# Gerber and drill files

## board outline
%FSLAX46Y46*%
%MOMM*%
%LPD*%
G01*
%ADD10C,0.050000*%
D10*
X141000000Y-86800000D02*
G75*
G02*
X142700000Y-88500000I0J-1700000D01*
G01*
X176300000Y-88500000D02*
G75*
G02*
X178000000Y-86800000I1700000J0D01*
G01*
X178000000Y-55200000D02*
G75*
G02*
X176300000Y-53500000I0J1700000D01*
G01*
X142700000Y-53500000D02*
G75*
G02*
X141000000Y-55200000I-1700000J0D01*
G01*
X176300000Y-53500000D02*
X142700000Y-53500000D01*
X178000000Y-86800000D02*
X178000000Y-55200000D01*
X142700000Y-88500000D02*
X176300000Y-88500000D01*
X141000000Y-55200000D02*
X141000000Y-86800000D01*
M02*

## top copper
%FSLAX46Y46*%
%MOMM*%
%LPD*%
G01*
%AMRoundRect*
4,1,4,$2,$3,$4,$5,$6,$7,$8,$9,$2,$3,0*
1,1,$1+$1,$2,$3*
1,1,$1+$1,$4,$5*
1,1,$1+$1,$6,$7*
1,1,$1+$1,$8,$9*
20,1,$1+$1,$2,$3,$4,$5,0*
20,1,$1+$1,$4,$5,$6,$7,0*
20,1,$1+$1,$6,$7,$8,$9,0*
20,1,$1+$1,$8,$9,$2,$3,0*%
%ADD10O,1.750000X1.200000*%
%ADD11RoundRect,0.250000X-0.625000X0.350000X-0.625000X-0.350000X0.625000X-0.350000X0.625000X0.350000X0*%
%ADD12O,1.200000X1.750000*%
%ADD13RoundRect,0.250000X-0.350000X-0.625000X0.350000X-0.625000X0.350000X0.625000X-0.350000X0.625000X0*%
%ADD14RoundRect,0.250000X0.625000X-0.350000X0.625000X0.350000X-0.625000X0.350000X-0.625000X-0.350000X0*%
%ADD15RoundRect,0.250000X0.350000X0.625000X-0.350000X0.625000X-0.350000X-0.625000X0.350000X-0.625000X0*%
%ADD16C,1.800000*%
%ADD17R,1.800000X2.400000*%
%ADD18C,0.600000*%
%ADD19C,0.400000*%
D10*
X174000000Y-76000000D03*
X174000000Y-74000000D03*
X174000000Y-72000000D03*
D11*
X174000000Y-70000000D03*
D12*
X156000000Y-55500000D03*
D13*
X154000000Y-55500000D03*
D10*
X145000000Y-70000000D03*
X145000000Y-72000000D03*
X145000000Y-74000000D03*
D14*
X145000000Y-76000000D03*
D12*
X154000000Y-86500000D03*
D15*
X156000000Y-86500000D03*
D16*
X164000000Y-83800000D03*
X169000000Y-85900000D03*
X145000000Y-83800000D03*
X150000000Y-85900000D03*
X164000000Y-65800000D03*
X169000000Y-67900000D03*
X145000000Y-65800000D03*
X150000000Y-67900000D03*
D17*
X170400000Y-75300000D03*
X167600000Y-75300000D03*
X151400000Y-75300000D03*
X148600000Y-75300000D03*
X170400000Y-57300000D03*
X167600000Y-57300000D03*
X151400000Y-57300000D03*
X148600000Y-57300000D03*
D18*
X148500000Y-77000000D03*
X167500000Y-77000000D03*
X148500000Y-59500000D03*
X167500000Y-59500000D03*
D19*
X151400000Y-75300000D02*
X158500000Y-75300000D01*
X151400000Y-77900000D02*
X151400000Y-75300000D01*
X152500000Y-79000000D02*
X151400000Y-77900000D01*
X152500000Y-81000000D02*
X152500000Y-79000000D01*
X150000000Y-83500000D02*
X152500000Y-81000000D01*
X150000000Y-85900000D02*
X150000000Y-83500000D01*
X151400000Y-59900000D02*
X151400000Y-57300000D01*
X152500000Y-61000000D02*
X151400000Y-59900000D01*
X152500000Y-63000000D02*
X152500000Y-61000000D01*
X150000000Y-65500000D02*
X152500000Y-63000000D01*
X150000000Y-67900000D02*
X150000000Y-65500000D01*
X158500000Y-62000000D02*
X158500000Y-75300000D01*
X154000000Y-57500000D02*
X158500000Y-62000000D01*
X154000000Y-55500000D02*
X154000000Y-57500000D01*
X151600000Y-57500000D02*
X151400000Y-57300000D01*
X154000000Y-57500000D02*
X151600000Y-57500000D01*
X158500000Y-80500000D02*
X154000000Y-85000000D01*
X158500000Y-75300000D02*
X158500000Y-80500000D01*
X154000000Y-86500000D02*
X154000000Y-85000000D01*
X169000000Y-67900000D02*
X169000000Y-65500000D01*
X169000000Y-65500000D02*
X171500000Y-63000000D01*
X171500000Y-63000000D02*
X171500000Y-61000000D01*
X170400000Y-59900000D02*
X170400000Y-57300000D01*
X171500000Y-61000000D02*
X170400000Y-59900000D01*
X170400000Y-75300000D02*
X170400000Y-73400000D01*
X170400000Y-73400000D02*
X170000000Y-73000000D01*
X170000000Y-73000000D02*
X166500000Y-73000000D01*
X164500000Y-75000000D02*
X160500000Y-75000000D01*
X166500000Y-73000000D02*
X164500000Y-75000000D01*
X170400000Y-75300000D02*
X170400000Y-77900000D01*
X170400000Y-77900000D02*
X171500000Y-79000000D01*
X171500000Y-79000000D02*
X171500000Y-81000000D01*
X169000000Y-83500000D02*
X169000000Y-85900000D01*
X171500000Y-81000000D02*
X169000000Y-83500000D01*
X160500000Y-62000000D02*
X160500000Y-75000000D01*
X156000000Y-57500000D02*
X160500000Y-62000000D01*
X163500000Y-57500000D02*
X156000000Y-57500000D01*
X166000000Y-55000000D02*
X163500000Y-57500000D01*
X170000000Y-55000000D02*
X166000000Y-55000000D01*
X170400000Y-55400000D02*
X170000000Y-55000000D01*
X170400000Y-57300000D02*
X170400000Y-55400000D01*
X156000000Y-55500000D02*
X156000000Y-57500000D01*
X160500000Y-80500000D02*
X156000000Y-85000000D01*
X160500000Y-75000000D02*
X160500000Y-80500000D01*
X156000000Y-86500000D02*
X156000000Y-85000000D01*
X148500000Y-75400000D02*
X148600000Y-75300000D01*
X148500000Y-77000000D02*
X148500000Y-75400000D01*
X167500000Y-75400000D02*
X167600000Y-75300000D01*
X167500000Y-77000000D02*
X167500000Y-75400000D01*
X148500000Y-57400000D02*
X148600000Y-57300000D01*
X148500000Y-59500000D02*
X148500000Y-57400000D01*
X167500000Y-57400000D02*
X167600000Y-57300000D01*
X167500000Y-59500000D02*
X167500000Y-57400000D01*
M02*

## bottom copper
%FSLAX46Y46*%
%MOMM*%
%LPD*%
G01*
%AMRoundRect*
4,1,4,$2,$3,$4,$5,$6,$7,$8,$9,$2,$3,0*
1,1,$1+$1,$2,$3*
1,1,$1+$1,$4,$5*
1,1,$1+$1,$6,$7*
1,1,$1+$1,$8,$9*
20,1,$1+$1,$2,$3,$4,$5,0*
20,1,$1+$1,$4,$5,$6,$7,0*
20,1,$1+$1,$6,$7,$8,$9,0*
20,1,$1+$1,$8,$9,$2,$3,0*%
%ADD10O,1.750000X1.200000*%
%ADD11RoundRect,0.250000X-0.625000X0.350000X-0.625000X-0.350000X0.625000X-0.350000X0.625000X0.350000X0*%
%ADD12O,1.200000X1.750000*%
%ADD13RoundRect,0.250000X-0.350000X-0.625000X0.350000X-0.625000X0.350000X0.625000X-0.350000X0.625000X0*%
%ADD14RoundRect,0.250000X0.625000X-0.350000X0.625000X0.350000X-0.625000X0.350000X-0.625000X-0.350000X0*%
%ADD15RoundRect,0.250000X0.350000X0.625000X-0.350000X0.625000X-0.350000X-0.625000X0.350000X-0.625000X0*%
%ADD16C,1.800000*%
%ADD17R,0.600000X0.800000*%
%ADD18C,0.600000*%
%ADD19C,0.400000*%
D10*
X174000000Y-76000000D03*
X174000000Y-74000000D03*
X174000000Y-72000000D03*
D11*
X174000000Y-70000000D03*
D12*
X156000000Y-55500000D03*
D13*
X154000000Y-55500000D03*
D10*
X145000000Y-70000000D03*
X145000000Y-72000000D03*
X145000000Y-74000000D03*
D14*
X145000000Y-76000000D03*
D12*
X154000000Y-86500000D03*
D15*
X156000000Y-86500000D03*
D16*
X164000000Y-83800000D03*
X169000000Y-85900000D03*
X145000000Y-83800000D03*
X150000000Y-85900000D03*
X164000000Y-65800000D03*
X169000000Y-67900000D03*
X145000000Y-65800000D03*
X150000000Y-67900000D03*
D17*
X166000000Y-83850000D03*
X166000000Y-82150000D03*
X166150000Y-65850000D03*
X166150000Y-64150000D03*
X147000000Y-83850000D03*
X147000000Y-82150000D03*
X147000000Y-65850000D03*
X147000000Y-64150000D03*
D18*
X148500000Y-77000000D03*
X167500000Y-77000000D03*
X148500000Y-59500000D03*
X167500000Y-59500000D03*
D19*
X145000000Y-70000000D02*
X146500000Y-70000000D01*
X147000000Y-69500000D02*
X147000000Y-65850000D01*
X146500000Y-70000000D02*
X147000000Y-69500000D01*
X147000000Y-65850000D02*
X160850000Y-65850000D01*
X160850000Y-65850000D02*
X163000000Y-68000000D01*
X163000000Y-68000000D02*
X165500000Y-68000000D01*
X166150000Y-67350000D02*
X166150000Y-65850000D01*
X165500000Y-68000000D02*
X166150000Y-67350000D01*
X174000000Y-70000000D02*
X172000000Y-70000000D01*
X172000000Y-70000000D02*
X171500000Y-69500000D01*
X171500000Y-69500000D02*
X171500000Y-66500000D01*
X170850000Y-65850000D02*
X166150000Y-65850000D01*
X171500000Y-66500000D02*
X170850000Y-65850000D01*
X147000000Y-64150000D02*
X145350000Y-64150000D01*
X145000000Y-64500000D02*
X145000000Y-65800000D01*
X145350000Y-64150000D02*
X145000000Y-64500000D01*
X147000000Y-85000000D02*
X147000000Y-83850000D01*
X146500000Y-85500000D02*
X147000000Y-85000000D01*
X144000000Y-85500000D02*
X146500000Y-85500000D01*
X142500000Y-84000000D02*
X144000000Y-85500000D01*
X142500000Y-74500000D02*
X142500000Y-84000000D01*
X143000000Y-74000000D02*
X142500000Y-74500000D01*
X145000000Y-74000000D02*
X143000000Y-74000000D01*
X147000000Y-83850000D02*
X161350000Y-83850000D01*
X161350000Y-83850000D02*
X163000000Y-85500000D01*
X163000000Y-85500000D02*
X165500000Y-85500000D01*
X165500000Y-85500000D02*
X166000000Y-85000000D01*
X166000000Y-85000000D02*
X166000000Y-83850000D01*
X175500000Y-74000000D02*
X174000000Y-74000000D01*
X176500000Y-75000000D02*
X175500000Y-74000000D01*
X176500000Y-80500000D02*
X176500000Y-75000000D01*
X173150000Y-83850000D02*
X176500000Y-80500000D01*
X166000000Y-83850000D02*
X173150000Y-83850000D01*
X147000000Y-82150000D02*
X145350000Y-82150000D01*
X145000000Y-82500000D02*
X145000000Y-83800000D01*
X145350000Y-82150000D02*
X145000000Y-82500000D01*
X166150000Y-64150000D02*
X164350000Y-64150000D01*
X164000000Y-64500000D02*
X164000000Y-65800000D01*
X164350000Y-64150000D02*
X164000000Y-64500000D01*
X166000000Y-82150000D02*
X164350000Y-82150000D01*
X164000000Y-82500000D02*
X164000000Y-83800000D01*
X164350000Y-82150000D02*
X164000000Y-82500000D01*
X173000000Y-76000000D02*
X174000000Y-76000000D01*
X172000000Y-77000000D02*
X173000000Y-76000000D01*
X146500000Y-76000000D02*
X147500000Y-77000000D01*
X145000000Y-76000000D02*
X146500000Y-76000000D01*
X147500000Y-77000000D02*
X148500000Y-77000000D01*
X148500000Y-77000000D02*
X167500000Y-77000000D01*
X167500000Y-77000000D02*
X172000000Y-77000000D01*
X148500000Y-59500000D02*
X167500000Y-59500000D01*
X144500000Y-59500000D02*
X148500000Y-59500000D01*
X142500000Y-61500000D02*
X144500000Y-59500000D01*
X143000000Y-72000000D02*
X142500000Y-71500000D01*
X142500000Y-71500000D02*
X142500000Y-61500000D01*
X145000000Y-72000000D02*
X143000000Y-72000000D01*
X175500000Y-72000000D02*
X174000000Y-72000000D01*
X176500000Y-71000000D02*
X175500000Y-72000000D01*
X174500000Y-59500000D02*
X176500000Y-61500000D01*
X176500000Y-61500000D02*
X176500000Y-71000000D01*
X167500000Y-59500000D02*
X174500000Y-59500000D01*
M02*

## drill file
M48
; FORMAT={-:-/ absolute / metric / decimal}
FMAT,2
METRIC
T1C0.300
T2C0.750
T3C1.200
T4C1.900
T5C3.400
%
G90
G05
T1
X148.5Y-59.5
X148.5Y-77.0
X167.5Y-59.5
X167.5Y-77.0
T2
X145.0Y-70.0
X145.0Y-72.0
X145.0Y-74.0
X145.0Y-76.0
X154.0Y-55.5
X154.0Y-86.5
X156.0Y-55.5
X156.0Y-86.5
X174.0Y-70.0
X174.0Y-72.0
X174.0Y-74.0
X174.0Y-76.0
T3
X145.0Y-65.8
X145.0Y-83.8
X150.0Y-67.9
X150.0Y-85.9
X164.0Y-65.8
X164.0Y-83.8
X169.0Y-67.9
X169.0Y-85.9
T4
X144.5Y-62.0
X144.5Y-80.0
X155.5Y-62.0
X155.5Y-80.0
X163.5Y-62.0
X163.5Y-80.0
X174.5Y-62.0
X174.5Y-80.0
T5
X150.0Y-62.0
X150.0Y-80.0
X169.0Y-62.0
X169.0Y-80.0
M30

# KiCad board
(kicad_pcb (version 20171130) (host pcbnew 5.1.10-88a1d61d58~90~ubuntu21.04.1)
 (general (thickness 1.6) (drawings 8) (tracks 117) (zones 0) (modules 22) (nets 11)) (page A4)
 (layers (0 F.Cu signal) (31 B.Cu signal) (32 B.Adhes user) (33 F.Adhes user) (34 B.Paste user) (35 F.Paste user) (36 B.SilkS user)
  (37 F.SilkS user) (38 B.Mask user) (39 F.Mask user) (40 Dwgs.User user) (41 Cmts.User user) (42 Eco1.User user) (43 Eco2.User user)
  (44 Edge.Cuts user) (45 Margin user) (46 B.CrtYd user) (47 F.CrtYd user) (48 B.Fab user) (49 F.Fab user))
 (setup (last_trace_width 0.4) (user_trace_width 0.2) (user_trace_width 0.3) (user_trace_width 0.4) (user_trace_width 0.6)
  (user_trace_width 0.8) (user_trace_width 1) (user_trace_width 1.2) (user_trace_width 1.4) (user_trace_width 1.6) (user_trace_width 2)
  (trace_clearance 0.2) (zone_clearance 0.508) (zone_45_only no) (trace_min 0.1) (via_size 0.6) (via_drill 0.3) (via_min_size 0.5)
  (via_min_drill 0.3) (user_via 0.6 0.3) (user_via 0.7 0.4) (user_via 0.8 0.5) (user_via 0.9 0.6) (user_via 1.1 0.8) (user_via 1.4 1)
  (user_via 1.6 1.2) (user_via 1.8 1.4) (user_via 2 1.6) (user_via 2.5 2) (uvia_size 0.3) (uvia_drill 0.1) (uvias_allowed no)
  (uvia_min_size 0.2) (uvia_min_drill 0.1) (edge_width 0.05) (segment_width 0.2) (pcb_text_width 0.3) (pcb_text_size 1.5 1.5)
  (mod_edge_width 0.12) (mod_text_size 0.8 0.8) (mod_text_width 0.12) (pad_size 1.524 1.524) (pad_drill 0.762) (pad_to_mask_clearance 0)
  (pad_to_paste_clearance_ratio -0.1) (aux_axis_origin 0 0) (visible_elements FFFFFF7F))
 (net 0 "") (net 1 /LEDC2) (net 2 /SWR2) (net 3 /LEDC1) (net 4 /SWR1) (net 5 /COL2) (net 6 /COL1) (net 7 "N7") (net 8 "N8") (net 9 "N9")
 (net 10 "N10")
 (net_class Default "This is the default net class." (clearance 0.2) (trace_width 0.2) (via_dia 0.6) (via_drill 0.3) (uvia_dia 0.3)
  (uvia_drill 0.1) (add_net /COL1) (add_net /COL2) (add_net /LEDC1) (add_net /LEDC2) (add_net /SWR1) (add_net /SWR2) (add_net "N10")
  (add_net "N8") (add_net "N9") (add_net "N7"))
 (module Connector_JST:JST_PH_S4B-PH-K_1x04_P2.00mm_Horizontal (layer B.Cu) (at 174 70 270)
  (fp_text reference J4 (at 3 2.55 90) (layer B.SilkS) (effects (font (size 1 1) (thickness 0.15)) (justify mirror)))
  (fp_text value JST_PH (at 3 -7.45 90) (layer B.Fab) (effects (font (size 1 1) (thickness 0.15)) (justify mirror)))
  (pad 4 thru_hole oval (at 6 0 270) (size 1.2 1.75) (drill 0.75) (layers *.Cu *.Mask) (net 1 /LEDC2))
  (pad 3 thru_hole oval (at 4 0 270) (size 1.2 1.75) (drill 0.75) (layers *.Cu *.Mask) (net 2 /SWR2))
  (pad 2 thru_hole oval (at 2 0 270) (size 1.2 1.75) (drill 0.75) (layers *.Cu *.Mask) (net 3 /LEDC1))
  (pad 1 thru_hole roundrect (at 0 0 270) (size 1.2 1.75) (drill 0.75) (layers *.Cu *.Mask) (roundrect_rratio 0.208333) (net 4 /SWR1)))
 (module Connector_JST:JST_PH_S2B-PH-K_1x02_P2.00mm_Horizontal (layer B.Cu) (at 154 55.5)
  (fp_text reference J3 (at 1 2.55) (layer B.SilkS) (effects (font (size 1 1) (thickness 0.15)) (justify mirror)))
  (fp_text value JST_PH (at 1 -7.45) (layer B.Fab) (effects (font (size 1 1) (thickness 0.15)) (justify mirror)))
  (pad 2 thru_hole oval (at 2 0) (size 1.2 1.75) (drill 0.75) (layers *.Cu *.Mask) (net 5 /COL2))
  (pad 1 thru_hole roundrect (at 0 0) (size 1.2 1.75) (drill 0.75) (layers *.Cu *.Mask) (roundrect_rratio 0.208333) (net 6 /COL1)))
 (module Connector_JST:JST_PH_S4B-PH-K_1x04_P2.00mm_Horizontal (layer B.Cu) (at 145 76 90)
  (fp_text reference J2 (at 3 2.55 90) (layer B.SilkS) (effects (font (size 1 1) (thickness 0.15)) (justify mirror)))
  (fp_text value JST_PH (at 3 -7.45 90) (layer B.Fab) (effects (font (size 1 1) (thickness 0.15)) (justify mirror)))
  (pad 4 thru_hole oval (at 6 0 90) (size 1.2 1.75) (drill 0.75) (layers *.Cu *.Mask) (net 4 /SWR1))
  (pad 3 thru_hole oval (at 4 0 90) (size 1.2 1.75) (drill 0.75) (layers *.Cu *.Mask) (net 3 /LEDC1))
  (pad 2 thru_hole oval (at 2 0 90) (size 1.2 1.75) (drill 0.75) (layers *.Cu *.Mask) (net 2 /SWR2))
  (pad 1 thru_hole roundrect (at 0 0 90) (size 1.2 1.75) (drill 0.75) (layers *.Cu *.Mask) (roundrect_rratio 0.208333) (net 1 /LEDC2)))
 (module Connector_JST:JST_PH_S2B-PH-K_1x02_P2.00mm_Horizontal (layer B.Cu) (at 156 86.5 180)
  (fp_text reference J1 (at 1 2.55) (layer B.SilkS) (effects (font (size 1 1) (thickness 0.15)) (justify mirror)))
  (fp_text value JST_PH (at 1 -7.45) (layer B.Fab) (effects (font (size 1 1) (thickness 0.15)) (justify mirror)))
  (pad 2 thru_hole oval (at 2 0 180) (size 1.2 1.75) (drill 0.75) (layers *.Cu *.Mask) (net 6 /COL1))
  (pad 1 thru_hole roundrect (at 0 0 180) (size 1.2 1.75) (drill 0.75) (layers *.Cu *.Mask) (roundrect_rratio 0.208333) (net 5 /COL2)))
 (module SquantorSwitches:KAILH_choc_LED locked (layer F.Cu) (at 169 80 180)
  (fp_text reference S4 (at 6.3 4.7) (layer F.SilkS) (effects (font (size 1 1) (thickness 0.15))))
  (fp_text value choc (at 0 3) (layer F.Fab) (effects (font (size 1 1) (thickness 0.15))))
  (pad 2 thru_hole circle (at 5 -3.8 180) (size 1.8 1.8) (drill 1.2) (layers *.Cu *.Mask) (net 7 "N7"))
  (pad 1 thru_hole circle (at 0 -5.9 180) (size 1.8 1.8) (drill 1.2) (layers *.Cu *.Mask) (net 5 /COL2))
  (pad "" np_thru_hole circle (at 5.5 0 180) (size 1.9 1.9) (drill 1.9) (layers *.Cu *.Mask))
  (pad "" np_thru_hole circle (at -5.5 0 180) (size 1.9 1.9) (drill 1.9) (layers *.Cu *.Mask))
  (pad "" np_thru_hole circle (at 0 0 180) (size 3.4 3.4) (drill 3.4) (layers *.Cu *.Mask)))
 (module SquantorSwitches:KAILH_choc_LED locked (layer F.Cu) (at 150 80 180)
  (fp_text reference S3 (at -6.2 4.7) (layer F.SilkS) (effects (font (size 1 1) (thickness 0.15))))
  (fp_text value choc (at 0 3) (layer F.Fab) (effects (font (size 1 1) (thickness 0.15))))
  (pad 2 thru_hole circle (at 5 -3.8 180) (size 1.8 1.8) (drill 1.2) (layers *.Cu *.Mask) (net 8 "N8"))
  (pad 1 thru_hole circle (at 0 -5.9 180) (size 1.8 1.8) (drill 1.2) (layers *.Cu *.Mask) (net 6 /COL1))
  (pad "" np_thru_hole circle (at 5.5 0 180) (size 1.9 1.9) (drill 1.9) (layers *.Cu *.Mask))
  (pad "" np_thru_hole circle (at -5.5 0 180) (size 1.9 1.9) (drill 1.9) (layers *.Cu *.Mask))
  (pad "" np_thru_hole circle (at 0 0 180) (size 3.4 3.4) (drill 3.4) (layers *.Cu *.Mask)))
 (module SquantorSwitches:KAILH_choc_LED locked (layer F.Cu) (at 169 62 180)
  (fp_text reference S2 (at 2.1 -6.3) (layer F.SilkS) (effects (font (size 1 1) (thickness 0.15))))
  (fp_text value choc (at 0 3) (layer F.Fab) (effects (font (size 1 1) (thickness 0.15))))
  (pad 2 thru_hole circle (at 5 -3.8 180) (size 1.8 1.8) (drill 1.2) (layers *.Cu *.Mask) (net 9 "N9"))
  (pad 1 thru_hole circle (at 0 -5.9 180) (size 1.8 1.8) (drill 1.2) (layers *.Cu *.Mask) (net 5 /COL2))
  (pad "" np_thru_hole circle (at 5.5 0 180) (size 1.9 1.9) (drill 1.9) (layers *.Cu *.Mask))
  (pad "" np_thru_hole circle (at -5.5 0 180) (size 1.9 1.9) (drill 1.9) (layers *.Cu *.Mask))
  (pad "" np_thru_hole circle (at 0 0 180) (size 3.4 3.4) (drill 3.4) (layers *.Cu *.Mask)))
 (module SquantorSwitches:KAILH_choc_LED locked (layer F.Cu) (at 150 62 180)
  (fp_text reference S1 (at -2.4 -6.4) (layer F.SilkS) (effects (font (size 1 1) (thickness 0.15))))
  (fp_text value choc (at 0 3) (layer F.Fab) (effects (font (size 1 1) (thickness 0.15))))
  (pad 2 thru_hole circle (at 5 -3.8 180) (size 1.8 1.8) (drill 1.2) (layers *.Cu *.Mask) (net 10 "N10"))
  (pad 1 thru_hole circle (at 0 -5.9 180) (size 1.8 1.8) (drill 1.2) (layers *.Cu *.Mask) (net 6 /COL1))
  (pad "" np_thru_hole circle (at 5.5 0 180) (size 1.9 1.9) (drill 1.9) (layers *.Cu *.Mask))
  (pad "" np_thru_hole circle (at -5.5 0 180) (size 1.9 1.9) (drill 1.9) (layers *.Cu *.Mask))
  (pad "" np_thru_hole circle (at 0 0 180) (size 3.4 3.4) (drill 3.4) (layers *.Cu *.Mask)))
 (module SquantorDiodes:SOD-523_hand (layer B.Cu) (at 166 83 90)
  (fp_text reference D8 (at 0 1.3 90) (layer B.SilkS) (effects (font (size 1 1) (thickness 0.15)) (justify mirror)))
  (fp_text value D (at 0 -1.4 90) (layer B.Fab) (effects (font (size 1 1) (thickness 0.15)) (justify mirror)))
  (pad 1 smd rect (at -0.85 0 90) (size 0.8 0.6) (layers B.Cu B.Paste B.Mask) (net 2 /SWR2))
  (pad 2 smd rect (at 0.85 0 90) (size 0.8 0.6) (layers B.Cu B.Paste B.Mask) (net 7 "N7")))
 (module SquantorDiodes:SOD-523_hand (layer B.Cu) (at 166.15 65 90)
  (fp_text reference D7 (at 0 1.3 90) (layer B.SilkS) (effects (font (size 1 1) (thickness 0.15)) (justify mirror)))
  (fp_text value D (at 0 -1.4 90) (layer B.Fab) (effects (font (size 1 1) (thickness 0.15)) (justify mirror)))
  (pad 1 smd rect (at -0.85 0 90) (size 0.8 0.6) (layers B.Cu B.Paste B.Mask) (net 4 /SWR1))
  (pad 2 smd rect (at 0.85 0 90) (size 0.8 0.6) (layers B.Cu B.Paste B.Mask) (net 9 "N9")))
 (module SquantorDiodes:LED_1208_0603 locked (layer F.Cu) (at 169 75.3)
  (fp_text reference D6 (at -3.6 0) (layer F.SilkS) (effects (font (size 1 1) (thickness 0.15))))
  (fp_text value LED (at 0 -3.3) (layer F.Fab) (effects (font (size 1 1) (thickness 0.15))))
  (pad 2 smd rect (at 1.4 0) (size 1.8 2.4) (layers F.Cu F.Paste F.Mask) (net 5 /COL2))
  (pad 1 smd rect (at -1.4 0) (size 1.8 2.4) (layers F.Cu F.Paste F.Mask) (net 1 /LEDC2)))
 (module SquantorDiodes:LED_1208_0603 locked (layer F.Cu) (at 150 75.3)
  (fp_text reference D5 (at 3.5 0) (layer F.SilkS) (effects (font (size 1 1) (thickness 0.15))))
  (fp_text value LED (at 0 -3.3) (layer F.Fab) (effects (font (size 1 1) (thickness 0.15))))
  (pad 2 smd rect (at 1.4 0) (size 1.8 2.4) (layers F.Cu F.Paste F.Mask) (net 6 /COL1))
  (pad 1 smd rect (at -1.4 0) (size 1.8 2.4) (layers F.Cu F.Paste F.Mask) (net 1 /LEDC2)))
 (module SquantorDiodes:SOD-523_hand (layer B.Cu) (at 147 83 90)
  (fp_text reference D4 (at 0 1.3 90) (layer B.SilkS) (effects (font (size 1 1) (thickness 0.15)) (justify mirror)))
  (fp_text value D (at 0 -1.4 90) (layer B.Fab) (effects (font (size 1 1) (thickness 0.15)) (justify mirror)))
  (pad 1 smd rect (at -0.85 0 90) (size 0.8 0.6) (layers B.Cu B.Paste B.Mask) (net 2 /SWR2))
  (pad 2 smd rect (at 0.85 0 90) (size 0.8 0.6) (layers B.Cu B.Paste B.Mask) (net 8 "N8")))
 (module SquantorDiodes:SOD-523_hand (layer B.Cu) (at 147 65 90)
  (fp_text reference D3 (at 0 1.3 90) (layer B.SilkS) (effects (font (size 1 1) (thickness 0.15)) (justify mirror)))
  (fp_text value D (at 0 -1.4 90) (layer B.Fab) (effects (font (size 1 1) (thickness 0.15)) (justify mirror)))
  (pad 1 smd rect (at -0.85 0 90) (size 0.8 0.6) (layers B.Cu B.Paste B.Mask) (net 4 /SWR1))
  (pad 2 smd rect (at 0.85 0 90) (size 0.8 0.6) (layers B.Cu B.Paste B.Mask) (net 10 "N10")))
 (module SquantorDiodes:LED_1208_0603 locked (layer F.Cu) (at 169 57.3)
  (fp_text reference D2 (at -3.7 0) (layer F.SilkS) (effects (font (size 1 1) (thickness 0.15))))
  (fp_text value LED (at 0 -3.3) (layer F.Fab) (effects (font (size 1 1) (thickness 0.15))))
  (pad 2 smd rect (at 1.4 0) (size 1.8 2.4) (layers F.Cu F.Paste F.Mask) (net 5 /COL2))
  (pad 1 smd rect (at -1.4 0) (size 1.8 2.4) (layers F.Cu F.Paste F.Mask) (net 3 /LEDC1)))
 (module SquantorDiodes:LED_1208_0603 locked (layer F.Cu) (at 150 57.3)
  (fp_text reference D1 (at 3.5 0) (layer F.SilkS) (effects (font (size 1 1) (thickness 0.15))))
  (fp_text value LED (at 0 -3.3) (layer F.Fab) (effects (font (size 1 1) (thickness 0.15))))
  (pad 2 smd rect (at 1.4 0) (size 1.8 2.4) (layers F.Cu F.Paste F.Mask) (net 6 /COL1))
  (pad 1 smd rect (at -1.4 0) (size 1.8 2.4) (layers F.Cu F.Paste F.Mask) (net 3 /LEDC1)))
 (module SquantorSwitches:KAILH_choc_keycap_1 (layer F.Cu) (at 169 80)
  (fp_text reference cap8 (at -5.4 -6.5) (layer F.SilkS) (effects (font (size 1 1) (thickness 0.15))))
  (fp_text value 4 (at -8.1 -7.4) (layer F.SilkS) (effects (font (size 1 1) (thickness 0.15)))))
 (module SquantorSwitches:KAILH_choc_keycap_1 (layer F.Cu) (at 150 80)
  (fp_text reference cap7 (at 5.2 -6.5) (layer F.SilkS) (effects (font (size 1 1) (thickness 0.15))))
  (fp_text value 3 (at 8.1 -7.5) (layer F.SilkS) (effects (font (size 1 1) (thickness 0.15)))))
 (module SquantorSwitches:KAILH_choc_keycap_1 (layer F.Cu) (at 169 62)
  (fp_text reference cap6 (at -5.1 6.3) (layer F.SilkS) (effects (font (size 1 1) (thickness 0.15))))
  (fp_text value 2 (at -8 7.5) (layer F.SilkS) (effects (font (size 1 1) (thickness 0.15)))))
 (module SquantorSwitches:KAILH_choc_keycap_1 (layer F.Cu) (at 150 62)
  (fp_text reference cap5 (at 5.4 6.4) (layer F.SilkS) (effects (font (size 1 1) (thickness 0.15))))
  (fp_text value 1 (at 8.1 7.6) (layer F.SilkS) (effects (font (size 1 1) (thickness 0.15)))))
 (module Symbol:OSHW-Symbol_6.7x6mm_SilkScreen (layer B.Cu) (at 159.5 71 180)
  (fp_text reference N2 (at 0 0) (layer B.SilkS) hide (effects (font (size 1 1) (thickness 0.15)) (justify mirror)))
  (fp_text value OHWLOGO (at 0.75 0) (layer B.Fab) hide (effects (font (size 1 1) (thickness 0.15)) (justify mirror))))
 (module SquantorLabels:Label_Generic (layer B.Cu) (at 160.3 74.7 180)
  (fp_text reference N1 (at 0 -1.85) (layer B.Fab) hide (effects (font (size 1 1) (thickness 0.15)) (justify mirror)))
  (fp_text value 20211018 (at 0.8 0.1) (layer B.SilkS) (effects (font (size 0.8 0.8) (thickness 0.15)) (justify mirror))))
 (gr_arc (start 141 88.5) (end 142.7 88.5) (angle -90) (layer Edge.Cuts) (width 0.05))
 (gr_arc (start 178 88.5) (end 178 86.8) (angle -90) (layer Edge.Cuts) (width 0.05))
 (gr_arc (start 178 53.5) (end 176.3 53.5) (angle -90) (layer Edge.Cuts) (width 0.05))
 (gr_arc (start 141 53.5) (end 141 55.2) (angle -90) (layer Edge.Cuts) (width 0.05))
 (gr_line (start 176.3 53.5) (end 142.7 53.5) (layer Edge.Cuts) (width 0.05))
 (gr_line (start 178 86.8) (end 178 55.2) (layer Edge.Cuts) (width 0.05))
 (gr_line (start 142.7 88.5) (end 176.3 88.5) (layer Edge.Cuts) (width 0.05))
 (gr_line (start 141 55.2) (end 141 86.8) (layer Edge.Cuts) (width 0.05))
 (segment (start 151.4 75.3) (end 158.5 75.3) (width 0.4) (layer F.Cu) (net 6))
 (segment (start 151.4 77.9) (end 151.4 75.3) (width 0.4) (layer F.Cu) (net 6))
 (segment (start 152.5 79) (end 151.4 77.9) (width 0.4) (layer F.Cu) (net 6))
 (segment (start 152.5 81) (end 152.5 79) (width 0.4) (layer F.Cu) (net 6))
 (segment (start 150 83.5) (end 152.5 81) (width 0.4) (layer F.Cu) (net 6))
 (segment (start 150 85.9) (end 150 83.5) (width 0.4) (layer F.Cu) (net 6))
 (segment (start 151.4 59.9) (end 151.4 57.3) (width 0.4) (layer F.Cu) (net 6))
 (segment (start 152.5 61) (end 151.4 59.9) (width 0.4) (layer F.Cu) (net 6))
 (segment (start 152.5 63) (end 152.5 61) (width 0.4) (layer F.Cu) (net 6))
 (segment (start 150 65.5) (end 152.5 63) (width 0.4) (layer F.Cu) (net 6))
 (segment (start 150 67.9) (end 150 65.5) (width 0.4) (layer F.Cu) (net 6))
 (segment (start 158.5 62) (end 158.5 75.3) (width 0.4) (layer F.Cu) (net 6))
 (segment (start 154 57.5) (end 158.5 62) (width 0.4) (layer F.Cu) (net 6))
 (segment (start 154 55.5) (end 154 57.5) (width 0.4) (layer F.Cu) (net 6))
 (segment (start 151.6 57.5) (end 151.4 57.3) (width 0.4) (layer F.Cu) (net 6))
 (segment (start 154 57.5) (end 151.6 57.5) (width 0.4) (layer F.Cu) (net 6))
 (segment (start 158.5 80.5) (end 154 85) (width 0.4) (layer F.Cu) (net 6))
 (segment (start 158.5 75.3) (end 158.5 80.5) (width 0.4) (layer F.Cu) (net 6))
 (segment (start 154 86.5) (end 154 85) (width 0.4) (layer F.Cu) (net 6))
 (segment (start 145 70) (end 146.5 70) (width 0.4) (layer B.Cu) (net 4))
 (segment (start 147 69.5) (end 147 65.85) (width 0.4) (layer B.Cu) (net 4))
 (segment (start 146.5 70) (end 147 69.5) (width 0.4) (layer B.Cu) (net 4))
 (segment (start 147 65.85) (end 160.85 65.85) (width 0.4) (layer B.Cu) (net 4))
 (segment (start 160.85 65.85) (end 163 68) (width 0.4) (layer B.Cu) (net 4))
 (segment (start 163 68) (end 165.5 68) (width 0.4) (layer B.Cu) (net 4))
 (segment (start 166.15 67.35) (end 166.15 65.85) (width 0.4) (layer B.Cu) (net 4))
 (segment (start 165.5 68) (end 166.15 67.35) (width 0.4) (layer B.Cu) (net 4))
 (segment (start 174 70) (end 172 70) (width 0.4) (layer B.Cu) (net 4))
 (segment (start 172 70) (end 171.5 69.5) (width 0.4) (layer B.Cu) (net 4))
 (segment (start 171.5 69.5) (end 171.5 66.5) (width 0.4) (layer B.Cu) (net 4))
 (segment (start 170.85 65.85) (end 166.15 65.85) (width 0.4) (layer B.Cu) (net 4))
 (segment (start 171.5 66.5) (end 170.85 65.85) (width 0.4) (layer B.Cu) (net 4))
 (segment (start 147 64.15) (end 145.35 64.15) (width 0.4) (layer B.Cu) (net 10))
 (segment (start 145 64.5) (end 145 65.8) (width 0.4) (layer B.Cu) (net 10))
 (segment (start 145.35 64.15) (end 145 64.5) (width 0.4) (layer B.Cu) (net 10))
 (segment (start 147 85) (end 147 83.85) (width 0.4) (layer B.Cu) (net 2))
 (segment (start 146.5 85.5) (end 147 85) (width 0.4) (layer B.Cu) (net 2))
 (segment (start 144 85.5) (end 146.5 85.5) (width 0.4) (layer B.Cu) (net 2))
 (segment (start 142.5 84) (end 144 85.5) (width 0.4) (layer B.Cu) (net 2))
 (segment (start 142.5 74.5) (end 142.5 84) (width 0.4) (layer B.Cu) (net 2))
 (segment (start 143 74) (end 142.5 74.5) (width 0.4) (layer B.Cu) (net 2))
 (segment (start 145 74) (end 143 74) (width 0.4) (layer B.Cu) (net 2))
 (segment (start 147 83.85) (end 161.35 83.85) (width 0.4) (layer B.Cu) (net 2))
 (segment (start 161.35 83.85) (end 163 85.5) (width 0.4) (layer B.Cu) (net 2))
 (segment (start 163 85.5) (end 165.5 85.5) (width 0.4) (layer B.Cu) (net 2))
 (segment (start 165.5 85.5) (end 166 85) (width 0.4) (layer B.Cu) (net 2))
 (segment (start 166 85) (end 166 83.85) (width 0.4) (layer B.Cu) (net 2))
 (segment (start 175.5 74) (end 174 74) (width 0.4) (layer B.Cu) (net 2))
 (segment (start 176.5 75) (end 175.5 74) (width 0.4) (layer B.Cu) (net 2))
 (segment (start 176.5 80.5) (end 176.5 75) (width 0.4) (layer B.Cu) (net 2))
 (segment (start 173.15 83.85) (end 176.5 80.5) (width 0.4) (layer B.Cu) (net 2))
 (segment (start 166 83.85) (end 173.15 83.85) (width 0.4) (layer B.Cu) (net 2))
 (segment (start 147 82.15) (end 145.35 82.15) (width 0.4) (layer B.Cu) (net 8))
 (segment (start 145 82.5) (end 145 83.8) (width 0.4) (layer B.Cu) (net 8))
 (segment (start 145.35 82.15) (end 145 82.5) (width 0.4) (layer B.Cu) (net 8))
 (segment (start 169 67.9) (end 169 65.5) (width 0.4) (layer F.Cu) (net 5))
 (segment (start 169 65.5) (end 171.5 63) (width 0.4) (layer F.Cu) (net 5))
 (segment (start 171.5 63) (end 171.5 61) (width 0.4) (layer F.Cu) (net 5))
 (segment (start 170.4 59.9) (end 170.4 57.3) (width 0.4) (layer F.Cu) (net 5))
 (segment (start 171.5 61) (end 170.4 59.9) (width 0.4) (layer F.Cu) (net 5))
 (segment (start 170.4 75.3) (end 170.4 73.4) (width 0.4) (layer F.Cu) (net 5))
 (segment (start 170.4 73.4) (end 170 73) (width 0.4) (layer F.Cu) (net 5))
 (segment (start 170 73) (end 166.5 73) (width 0.4) (layer F.Cu) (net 5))
 (segment (start 164.5 75) (end 160.5 75) (width 0.4) (layer F.Cu) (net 5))
 (segment (start 166.5 73) (end 164.5 75) (width 0.4) (layer F.Cu) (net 5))
 (segment (start 170.4 75.3) (end 170.4 77.9) (width 0.4) (layer F.Cu) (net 5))
 (segment (start 170.4 77.9) (end 171.5 79) (width 0.4) (layer F.Cu) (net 5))
 (segment (start 171.5 79) (end 171.5 81) (width 0.4) (layer F.Cu) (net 5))
 (segment (start 169 83.5) (end 169 85.9) (width 0.4) (layer F.Cu) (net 5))
 (segment (start 171.5 81) (end 169 83.5) (width 0.4) (layer F.Cu) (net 5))
 (segment (start 160.5 62) (end 160.5 75) (width 0.4) (layer F.Cu) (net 5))
 (segment (start 156 57.5) (end 160.5 62) (width 0.4) (layer F.Cu) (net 5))
 (segment (start 163.5 57.5) (end 156 57.5) (width 0.4) (layer F.Cu) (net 5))
 (segment (start 166 55) (end 163.5 57.5) (width 0.4) (layer F.Cu) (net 5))
 (segment (start 170 55) (end 166 55) (width 0.4) (layer F.Cu) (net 5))
 (segment (start 170.4 55.4) (end 170 55) (width 0.4) (layer F.Cu) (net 5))
 (segment (start 170.4 57.3) (end 170.4 55.4) (width 0.4) (layer F.Cu) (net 5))
 (segment (start 156 55.5) (end 156 57.5) (width 0.4) (layer F.Cu) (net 5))
 (segment (start 160.5 80.5) (end 156 85) (width 0.4) (layer F.Cu) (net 5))
 (segment (start 160.5 75) (end 160.5 80.5) (width 0.4) (layer F.Cu) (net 5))
 (segment (start 156 86.5) (end 156 85) (width 0.4) (layer F.Cu) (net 5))
 (segment (start 166.15 64.15) (end 164.35 64.15) (width 0.4) (layer B.Cu) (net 9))
 (segment (start 164 64.5) (end 164 65.8) (width 0.4) (layer B.Cu) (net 9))
 (segment (start 164.35 64.15) (end 164 64.5) (width 0.4) (layer B.Cu) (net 9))
 (segment (start 166 82.15) (end 164.35 82.15) (width 0.4) (layer B.Cu) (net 7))
 (segment (start 164 82.5) (end 164 83.8) (width 0.4) (layer B.Cu) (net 7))
 (segment (start 164.35 82.15) (end 164 82.5) (width 0.4) (layer B.Cu) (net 7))
 (segment (start 173 76) (end 174 76) (width 0.4) (layer B.Cu) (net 1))
 (segment (start 172 77) (end 173 76) (width 0.4) (layer B.Cu) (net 1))
 (segment (start 146.5 76) (end 147.5 77) (width 0.4) (layer B.Cu) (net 1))
 (segment (start 145 76) (end 146.5 76) (width 0.4) (layer B.Cu) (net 1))
 (via (at 148.5 77) (size 0.6) (drill 0.3) (layers F.Cu B.Cu) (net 1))
 (segment (start 147.5 77) (end 148.5 77) (width 0.4) (layer B.Cu) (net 1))
 (segment (start 148.5 75.4) (end 148.6 75.3) (width 0.4) (layer F.Cu) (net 1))
 (segment (start 148.5 77) (end 148.5 75.4) (width 0.4) (layer F.Cu) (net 1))
 (via (at 167.5 77) (size 0.6) (drill 0.3) (layers F.Cu B.Cu) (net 1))
 (segment (start 148.5 77) (end 167.5 77) (width 0.4) (layer B.Cu) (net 1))
 (segment (start 167.5 77) (end 172 77) (width 0.4) (layer B.Cu) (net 1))
 (segment (start 167.5 75.4) (end 167.6 75.3) (width 0.4) (layer F.Cu) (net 1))
 (segment (start 167.5 77) (end 167.5 75.4) (width 0.4) (layer F.Cu) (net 1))
 (via (at 148.5 59.5) (size 0.6) (drill 0.3) (layers F.Cu B.Cu) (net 3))
 (segment (start 148.5 57.4) (end 148.6 57.3) (width 0.4) (layer F.Cu) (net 3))
 (segment (start 148.5 59.5) (end 148.5 57.4) (width 0.4) (layer F.Cu) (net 3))
 (via (at 167.5 59.5) (size 0.6) (drill 0.3) (layers F.Cu B.Cu) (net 3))
 (segment (start 148.5 59.5) (end 167.5 59.5) (width 0.4) (layer B.Cu) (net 3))
 (segment (start 167.5 57.4) (end 167.6 57.3) (width 0.4) (layer F.Cu) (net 3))
 (segment (start 167.5 59.5) (end 167.5 57.4) (width 0.4) (layer F.Cu) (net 3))
 (segment (start 144.5 59.5) (end 148.5 59.5) (width 0.4) (layer B.Cu) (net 3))
 (segment (start 142.5 61.5) (end 144.5 59.5) (width 0.4) (layer B.Cu) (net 3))
 (segment (start 143 72) (end 142.5 71.5) (width 0.4) (layer B.Cu) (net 3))
 (segment (start 142.5 71.5) (end 142.5 61.5) (width 0.4) (layer B.Cu) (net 3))
 (segment (start 145 72) (end 143 72) (width 0.4) (layer B.Cu) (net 3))
 (segment (start 175.5 72) (end 174 72) (width 0.4) (layer B.Cu) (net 3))
 (segment (start 176.5 71) (end 175.5 72) (width 0.4) (layer B.Cu) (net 3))
 (segment (start 174.5 59.5) (end 176.5 61.5) (width 0.4) (layer B.Cu) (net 3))
 (segment (start 176.5 61.5) (end 176.5 71) (width 0.4) (layer B.Cu) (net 3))
 (segment (start 167.5 59.5) (end 174.5 59.5) (width 0.4) (layer B.Cu) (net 3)))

